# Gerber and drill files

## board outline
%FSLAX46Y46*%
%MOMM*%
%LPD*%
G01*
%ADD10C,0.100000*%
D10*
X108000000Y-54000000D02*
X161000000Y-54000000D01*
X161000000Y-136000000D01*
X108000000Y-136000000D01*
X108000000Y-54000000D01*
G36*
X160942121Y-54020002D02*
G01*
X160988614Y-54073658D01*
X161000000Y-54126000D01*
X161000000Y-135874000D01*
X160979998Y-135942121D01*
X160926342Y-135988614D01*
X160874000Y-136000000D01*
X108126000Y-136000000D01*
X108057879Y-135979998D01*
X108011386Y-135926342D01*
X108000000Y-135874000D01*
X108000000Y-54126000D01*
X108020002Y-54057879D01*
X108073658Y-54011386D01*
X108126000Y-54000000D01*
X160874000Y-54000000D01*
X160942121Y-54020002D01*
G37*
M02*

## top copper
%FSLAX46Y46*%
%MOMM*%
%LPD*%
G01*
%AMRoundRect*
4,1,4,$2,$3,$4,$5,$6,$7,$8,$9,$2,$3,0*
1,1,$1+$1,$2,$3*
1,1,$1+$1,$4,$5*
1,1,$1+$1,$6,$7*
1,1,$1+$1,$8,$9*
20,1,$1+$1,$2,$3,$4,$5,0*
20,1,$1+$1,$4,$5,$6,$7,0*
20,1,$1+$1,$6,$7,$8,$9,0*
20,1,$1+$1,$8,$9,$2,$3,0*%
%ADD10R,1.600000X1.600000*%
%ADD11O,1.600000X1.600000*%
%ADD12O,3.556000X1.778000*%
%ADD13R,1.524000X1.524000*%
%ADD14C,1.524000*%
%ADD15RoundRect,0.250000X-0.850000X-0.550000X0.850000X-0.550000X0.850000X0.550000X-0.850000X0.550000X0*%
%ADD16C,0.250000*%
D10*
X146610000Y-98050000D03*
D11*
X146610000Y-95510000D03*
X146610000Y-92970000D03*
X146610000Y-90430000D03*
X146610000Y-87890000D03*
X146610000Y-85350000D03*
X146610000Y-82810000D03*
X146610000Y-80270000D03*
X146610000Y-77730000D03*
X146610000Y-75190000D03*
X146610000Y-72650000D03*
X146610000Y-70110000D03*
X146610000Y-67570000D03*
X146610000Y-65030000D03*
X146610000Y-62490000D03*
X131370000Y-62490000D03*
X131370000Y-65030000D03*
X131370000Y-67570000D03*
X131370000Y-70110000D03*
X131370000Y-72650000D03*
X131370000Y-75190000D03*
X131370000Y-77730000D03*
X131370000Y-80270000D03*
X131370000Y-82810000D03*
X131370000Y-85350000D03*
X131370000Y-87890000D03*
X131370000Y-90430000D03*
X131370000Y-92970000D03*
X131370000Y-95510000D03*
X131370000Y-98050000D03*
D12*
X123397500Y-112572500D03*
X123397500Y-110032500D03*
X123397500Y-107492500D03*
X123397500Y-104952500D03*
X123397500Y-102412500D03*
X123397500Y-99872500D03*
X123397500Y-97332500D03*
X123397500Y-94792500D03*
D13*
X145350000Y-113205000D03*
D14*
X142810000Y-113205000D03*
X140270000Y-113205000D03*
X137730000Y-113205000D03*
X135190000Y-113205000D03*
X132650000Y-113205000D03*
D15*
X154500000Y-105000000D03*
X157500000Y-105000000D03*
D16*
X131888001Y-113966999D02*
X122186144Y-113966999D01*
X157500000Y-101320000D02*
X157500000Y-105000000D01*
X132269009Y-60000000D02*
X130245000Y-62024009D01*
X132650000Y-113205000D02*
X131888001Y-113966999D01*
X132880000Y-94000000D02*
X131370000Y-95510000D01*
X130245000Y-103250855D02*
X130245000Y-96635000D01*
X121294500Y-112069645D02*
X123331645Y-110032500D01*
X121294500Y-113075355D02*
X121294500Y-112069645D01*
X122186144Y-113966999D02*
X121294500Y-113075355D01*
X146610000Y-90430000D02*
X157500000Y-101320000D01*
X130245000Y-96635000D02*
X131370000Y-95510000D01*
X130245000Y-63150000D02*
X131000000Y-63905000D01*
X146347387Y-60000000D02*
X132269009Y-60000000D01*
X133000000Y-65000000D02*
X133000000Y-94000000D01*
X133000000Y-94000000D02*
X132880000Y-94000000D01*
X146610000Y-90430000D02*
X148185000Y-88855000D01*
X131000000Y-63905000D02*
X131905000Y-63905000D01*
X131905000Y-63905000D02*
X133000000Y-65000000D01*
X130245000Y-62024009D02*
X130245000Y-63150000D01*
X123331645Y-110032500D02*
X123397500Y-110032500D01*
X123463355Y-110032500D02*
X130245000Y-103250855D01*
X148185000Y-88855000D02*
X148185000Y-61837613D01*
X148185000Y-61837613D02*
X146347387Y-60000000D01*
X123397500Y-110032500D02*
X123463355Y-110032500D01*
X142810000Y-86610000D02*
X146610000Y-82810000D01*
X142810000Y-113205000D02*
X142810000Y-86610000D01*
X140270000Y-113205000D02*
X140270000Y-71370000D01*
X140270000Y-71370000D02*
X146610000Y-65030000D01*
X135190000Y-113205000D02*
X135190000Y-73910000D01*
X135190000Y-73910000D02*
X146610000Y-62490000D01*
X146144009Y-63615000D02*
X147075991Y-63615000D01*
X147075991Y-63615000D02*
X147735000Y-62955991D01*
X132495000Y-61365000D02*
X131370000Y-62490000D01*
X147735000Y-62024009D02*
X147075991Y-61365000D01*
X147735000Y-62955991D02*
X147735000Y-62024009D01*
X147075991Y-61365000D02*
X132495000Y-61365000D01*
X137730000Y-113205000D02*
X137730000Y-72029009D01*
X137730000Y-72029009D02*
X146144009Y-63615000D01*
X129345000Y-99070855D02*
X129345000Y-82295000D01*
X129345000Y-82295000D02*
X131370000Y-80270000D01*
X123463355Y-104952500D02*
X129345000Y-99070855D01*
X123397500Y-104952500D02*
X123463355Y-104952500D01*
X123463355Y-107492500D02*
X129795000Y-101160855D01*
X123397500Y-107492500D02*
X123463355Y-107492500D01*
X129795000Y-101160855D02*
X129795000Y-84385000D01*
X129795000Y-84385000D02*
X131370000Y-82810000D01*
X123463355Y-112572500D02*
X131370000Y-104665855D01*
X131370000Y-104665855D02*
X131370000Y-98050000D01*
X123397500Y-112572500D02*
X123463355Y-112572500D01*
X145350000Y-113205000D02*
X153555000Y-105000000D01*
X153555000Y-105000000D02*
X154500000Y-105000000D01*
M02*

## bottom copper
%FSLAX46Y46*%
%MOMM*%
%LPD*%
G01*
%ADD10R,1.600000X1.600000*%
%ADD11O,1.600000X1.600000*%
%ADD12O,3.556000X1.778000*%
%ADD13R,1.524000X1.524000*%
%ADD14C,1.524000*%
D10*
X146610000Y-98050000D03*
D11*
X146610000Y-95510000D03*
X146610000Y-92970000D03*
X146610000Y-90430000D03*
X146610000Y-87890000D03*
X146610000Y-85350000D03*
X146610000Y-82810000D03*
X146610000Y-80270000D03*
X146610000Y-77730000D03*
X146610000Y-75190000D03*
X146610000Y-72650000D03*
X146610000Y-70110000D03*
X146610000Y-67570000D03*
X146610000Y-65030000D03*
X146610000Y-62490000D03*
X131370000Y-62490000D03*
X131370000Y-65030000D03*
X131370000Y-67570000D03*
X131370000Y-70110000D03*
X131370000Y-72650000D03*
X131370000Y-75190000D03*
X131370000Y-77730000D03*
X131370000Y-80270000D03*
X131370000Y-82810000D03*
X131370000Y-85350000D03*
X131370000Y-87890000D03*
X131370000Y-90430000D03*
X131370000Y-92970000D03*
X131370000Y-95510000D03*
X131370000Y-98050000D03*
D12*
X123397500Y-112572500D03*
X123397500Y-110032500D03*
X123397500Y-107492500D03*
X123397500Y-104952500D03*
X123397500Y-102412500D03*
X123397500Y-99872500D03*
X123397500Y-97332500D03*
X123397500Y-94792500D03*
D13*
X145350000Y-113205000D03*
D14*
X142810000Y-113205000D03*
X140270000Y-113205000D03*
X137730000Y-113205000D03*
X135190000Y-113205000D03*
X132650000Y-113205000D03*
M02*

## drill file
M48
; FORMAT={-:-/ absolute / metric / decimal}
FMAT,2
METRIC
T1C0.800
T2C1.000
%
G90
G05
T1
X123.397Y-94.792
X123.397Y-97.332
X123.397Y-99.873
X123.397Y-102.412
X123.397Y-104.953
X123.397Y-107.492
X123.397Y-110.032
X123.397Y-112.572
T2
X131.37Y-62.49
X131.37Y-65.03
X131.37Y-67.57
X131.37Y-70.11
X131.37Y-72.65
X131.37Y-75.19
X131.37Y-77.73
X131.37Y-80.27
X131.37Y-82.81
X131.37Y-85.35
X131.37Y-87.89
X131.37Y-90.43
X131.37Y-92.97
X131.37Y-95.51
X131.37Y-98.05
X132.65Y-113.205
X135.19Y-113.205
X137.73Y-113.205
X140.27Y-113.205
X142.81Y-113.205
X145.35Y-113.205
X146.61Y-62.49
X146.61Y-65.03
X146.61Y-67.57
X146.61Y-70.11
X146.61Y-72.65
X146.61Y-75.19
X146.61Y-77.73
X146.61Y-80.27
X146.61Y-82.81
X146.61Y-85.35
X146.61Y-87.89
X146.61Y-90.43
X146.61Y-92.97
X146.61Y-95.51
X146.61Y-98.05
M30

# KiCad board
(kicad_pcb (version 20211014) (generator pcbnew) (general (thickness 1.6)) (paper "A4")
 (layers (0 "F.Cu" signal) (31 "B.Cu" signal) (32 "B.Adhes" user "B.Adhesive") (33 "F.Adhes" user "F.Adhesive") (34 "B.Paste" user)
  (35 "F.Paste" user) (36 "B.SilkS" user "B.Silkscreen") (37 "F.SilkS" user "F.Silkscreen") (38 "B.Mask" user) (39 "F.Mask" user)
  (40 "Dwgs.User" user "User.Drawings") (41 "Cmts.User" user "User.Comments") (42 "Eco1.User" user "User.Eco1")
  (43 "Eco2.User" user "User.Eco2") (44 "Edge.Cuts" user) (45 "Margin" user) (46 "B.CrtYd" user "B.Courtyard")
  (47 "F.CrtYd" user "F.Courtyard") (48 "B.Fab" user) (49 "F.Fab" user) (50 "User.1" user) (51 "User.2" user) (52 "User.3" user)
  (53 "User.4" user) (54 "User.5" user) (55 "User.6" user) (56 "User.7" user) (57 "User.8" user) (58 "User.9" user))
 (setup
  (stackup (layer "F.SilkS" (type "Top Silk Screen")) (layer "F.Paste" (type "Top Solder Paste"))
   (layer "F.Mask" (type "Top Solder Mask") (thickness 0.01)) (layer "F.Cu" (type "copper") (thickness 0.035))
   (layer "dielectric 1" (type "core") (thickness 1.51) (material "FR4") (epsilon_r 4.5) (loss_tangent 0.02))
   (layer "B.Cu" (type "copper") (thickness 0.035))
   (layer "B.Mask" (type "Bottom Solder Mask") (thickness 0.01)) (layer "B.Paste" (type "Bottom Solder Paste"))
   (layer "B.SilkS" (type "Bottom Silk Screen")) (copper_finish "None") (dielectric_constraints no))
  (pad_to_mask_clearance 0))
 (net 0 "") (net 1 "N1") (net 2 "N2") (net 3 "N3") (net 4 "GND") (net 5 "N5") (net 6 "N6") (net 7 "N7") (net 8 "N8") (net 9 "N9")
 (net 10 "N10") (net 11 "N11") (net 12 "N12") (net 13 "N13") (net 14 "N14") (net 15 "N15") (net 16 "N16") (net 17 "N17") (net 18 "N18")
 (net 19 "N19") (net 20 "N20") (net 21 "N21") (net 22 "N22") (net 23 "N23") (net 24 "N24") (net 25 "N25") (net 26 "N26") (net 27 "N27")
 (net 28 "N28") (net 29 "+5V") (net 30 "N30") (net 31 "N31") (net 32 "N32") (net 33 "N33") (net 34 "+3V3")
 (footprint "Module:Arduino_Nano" (layer "F.Cu") (at 146.61 98.05 180)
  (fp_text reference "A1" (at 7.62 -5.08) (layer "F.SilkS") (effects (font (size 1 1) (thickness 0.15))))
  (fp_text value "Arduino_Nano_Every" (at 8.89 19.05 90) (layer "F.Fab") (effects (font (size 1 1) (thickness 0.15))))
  (pad "1" thru_hole rect (at 0 0 180) (size 1.6 1.6) (drill 1) (layers *.Cu *.Mask) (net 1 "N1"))
  (pad "2" thru_hole oval (at 0 2.54 180) (size 1.6 1.6) (drill 1) (layers *.Cu *.Mask) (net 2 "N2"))
  (pad "3" thru_hole oval (at 0 5.08 180) (size 1.6 1.6) (drill 1) (layers *.Cu *.Mask) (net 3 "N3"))
  (pad "4" thru_hole oval (at 0 7.62 180) (size 1.6 1.6) (drill 1) (layers *.Cu *.Mask) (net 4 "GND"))
  (pad "5" thru_hole oval (at 0 10.16 180) (size 1.6 1.6) (drill 1) (layers *.Cu *.Mask) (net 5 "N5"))
  (pad "6" thru_hole oval (at 0 12.7 180) (size 1.6 1.6) (drill 1) (layers *.Cu *.Mask) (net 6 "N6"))
  (pad "7" thru_hole oval (at 0 15.24 180) (size 1.6 1.6) (drill 1) (layers *.Cu *.Mask) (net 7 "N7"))
  (pad "8" thru_hole oval (at 0 17.78 180) (size 1.6 1.6) (drill 1) (layers *.Cu *.Mask) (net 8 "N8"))
  (pad "9" thru_hole oval (at 0 20.32 180) (size 1.6 1.6) (drill 1) (layers *.Cu *.Mask) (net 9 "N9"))
  (pad "10" thru_hole oval (at 0 22.86 180) (size 1.6 1.6) (drill 1) (layers *.Cu *.Mask) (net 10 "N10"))
  (pad "11" thru_hole oval (at 0 25.4 180) (size 1.6 1.6) (drill 1) (layers *.Cu *.Mask) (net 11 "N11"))
  (pad "12" thru_hole oval (at 0 27.94 180) (size 1.6 1.6) (drill 1) (layers *.Cu *.Mask) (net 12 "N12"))
  (pad "13" thru_hole oval (at 0 30.48 180) (size 1.6 1.6) (drill 1) (layers *.Cu *.Mask) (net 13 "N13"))
  (pad "14" thru_hole oval (at 0 33.02 180) (size 1.6 1.6) (drill 1) (layers *.Cu *.Mask) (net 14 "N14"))
  (pad "15" thru_hole oval (at 0 35.56 180) (size 1.6 1.6) (drill 1) (layers *.Cu *.Mask) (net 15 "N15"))
  (pad "16" thru_hole oval (at 15.24 35.56 180) (size 1.6 1.6) (drill 1) (layers *.Cu *.Mask) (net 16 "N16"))
  (pad "17" thru_hole oval (at 15.24 33.02 180) (size 1.6 1.6) (drill 1) (layers *.Cu *.Mask) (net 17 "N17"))
  (pad "18" thru_hole oval (at 15.24 30.48 180) (size 1.6 1.6) (drill 1) (layers *.Cu *.Mask) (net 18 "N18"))
  (pad "19" thru_hole oval (at 15.24 27.94 180) (size 1.6 1.6) (drill 1) (layers *.Cu *.Mask) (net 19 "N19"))
  (pad "20" thru_hole oval (at 15.24 25.4 180) (size 1.6 1.6) (drill 1) (layers *.Cu *.Mask) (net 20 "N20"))
  (pad "21" thru_hole oval (at 15.24 22.86 180) (size 1.6 1.6) (drill 1) (layers *.Cu *.Mask) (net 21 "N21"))
  (pad "22" thru_hole oval (at 15.24 20.32 180) (size 1.6 1.6) (drill 1) (layers *.Cu *.Mask) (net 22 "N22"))
  (pad "23" thru_hole oval (at 15.24 17.78 180) (size 1.6 1.6) (drill 1) (layers *.Cu *.Mask) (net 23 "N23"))
  (pad "24" thru_hole oval (at 15.24 15.24 180) (size 1.6 1.6) (drill 1) (layers *.Cu *.Mask) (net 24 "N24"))
  (pad "25" thru_hole oval (at 15.24 12.7 180) (size 1.6 1.6) (drill 1) (layers *.Cu *.Mask) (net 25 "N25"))
  (pad "26" thru_hole oval (at 15.24 10.16 180) (size 1.6 1.6) (drill 1) (layers *.Cu *.Mask) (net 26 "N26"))
  (pad "27" thru_hole oval (at 15.24 7.62 180) (size 1.6 1.6) (drill 1) (layers *.Cu *.Mask) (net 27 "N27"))
  (pad "28" thru_hole oval (at 15.24 5.08 180) (size 1.6 1.6) (drill 1) (layers *.Cu *.Mask) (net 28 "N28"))
  (pad "29" thru_hole oval (at 15.24 2.54 180) (size 1.6 1.6) (drill 1) (layers *.Cu *.Mask) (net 4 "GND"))
  (pad "30" thru_hole oval (at 15.24 0 180) (size 1.6 1.6) (drill 1) (layers *.Cu *.Mask) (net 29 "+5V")))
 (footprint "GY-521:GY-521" (layer "F.Cu") (at 114.5075 103.6825 180)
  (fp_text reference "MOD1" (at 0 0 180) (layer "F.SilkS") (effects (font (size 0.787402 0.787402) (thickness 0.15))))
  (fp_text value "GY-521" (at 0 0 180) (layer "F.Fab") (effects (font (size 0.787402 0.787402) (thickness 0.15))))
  (pad "1" thru_hole oval locked (at -8.89 -8.89 180) (size 3.556 1.778) (drill 0.8) (layers *.Cu *.Mask) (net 29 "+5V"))
  (pad "2" thru_hole oval locked (at -8.89 -6.35 180) (size 3.556 1.778) (drill 0.8) (layers *.Cu *.Mask) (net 4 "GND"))
  (pad "3" thru_hole oval locked (at -8.89 -3.81 180) (size 3.556 1.778) (drill 0.8) (layers *.Cu *.Mask) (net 24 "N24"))
  (pad "4" thru_hole oval locked (at -8.89 -1.27 180) (size 3.556 1.778) (drill 0.8) (layers *.Cu *.Mask) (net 23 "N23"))
  (pad "5" thru_hole oval locked (at -8.89 1.27 180) (size 3.556 1.778) (drill 0.8) (layers *.Cu *.Mask) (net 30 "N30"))
  (pad "6" thru_hole oval locked (at -8.89 3.81 180) (size 3.556 1.778) (drill 0.8) (layers *.Cu *.Mask) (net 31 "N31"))
  (pad "7" thru_hole oval locked (at -8.89 6.35 180) (size 3.556 1.778) (drill 0.8) (layers *.Cu *.Mask) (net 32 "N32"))
  (pad "8" thru_hole oval locked (at -8.89 8.89 180) (size 3.556 1.778) (drill 0.8) (layers *.Cu *.Mask) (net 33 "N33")))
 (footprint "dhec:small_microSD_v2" (layer "F.Cu") (at 138.365 110.03)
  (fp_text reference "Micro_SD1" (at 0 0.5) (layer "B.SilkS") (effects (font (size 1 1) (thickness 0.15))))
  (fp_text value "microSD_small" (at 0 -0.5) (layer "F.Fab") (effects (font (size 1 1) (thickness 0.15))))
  (pad "1" thru_hole rect locked (at 6.985 3.175) (size 1.524 1.524) (drill 1) (layers *.Cu *.Mask) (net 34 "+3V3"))
  (pad "2" thru_hole circle locked (at 4.445 3.175) (size 1.524 1.524) (drill 1) (layers *.Cu *.Mask) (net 7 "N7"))
  (pad "3" thru_hole circle locked (at 1.905 3.175) (size 1.524 1.524) (drill 1) (layers *.Cu *.Mask) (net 14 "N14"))
  (pad "4" thru_hole circle locked (at -0.635 3.175) (size 1.524 1.524) (drill 1) (layers *.Cu *.Mask) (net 16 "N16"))
  (pad "5" thru_hole circle locked (at -3.175 3.175) (size 1.524 1.524) (drill 1) (layers *.Cu *.Mask) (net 15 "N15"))
  (pad "6" thru_hole circle locked (at -5.715 3.175) (size 1.524 1.524) (drill 1) (layers *.Cu *.Mask) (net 4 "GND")))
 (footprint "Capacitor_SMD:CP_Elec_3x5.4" (layer "F.Cu") (at 156 105)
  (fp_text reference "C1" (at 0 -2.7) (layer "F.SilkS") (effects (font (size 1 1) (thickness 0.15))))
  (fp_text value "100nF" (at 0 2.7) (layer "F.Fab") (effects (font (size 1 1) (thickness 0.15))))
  (pad "1" smd roundrect (at -1.5 0) (size 2.2 1.6) (layers "F.Cu" "F.Paste" "F.Mask") (roundrect_rratio 0.15625) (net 34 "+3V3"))
  (pad "2" smd roundrect (at 1.5 0) (size 2.2 1.6) (layers "F.Cu" "F.Paste" "F.Mask") (roundrect_rratio 0.15625) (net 4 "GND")))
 (gr_rect (start 108 54) (end 161 136) (layer "Edge.Cuts") (width 0.1) (fill none))
 (segment (start 131.888001 113.966999) (end 122.186144 113.966999) (width 0.25) (layer "F.Cu") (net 4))
 (segment (start 157.5 101.32) (end 157.5 105) (width 0.25) (layer "F.Cu") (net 4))
 (segment (start 132.269009 60) (end 130.245 62.024009) (width 0.25) (layer "F.Cu") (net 4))
 (segment (start 132.65 113.205) (end 131.888001 113.966999) (width 0.25) (layer "F.Cu") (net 4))
 (segment (start 132.88 94) (end 131.37 95.51) (width 0.25) (layer "F.Cu") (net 4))
 (segment (start 130.245 103.250855) (end 130.245 96.635) (width 0.25) (layer "F.Cu") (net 4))
 (segment (start 121.2945 112.069645) (end 123.331645 110.0325) (width 0.25) (layer "F.Cu") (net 4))
 (segment (start 121.2945 113.075355) (end 121.2945 112.069645) (width 0.25) (layer "F.Cu") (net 4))
 (segment (start 122.186144 113.966999) (end 121.2945 113.075355) (width 0.25) (layer "F.Cu") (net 4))
 (segment (start 146.61 90.43) (end 157.5 101.32) (width 0.25) (layer "F.Cu") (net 4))
 (segment (start 130.245 96.635) (end 131.37 95.51) (width 0.25) (layer "F.Cu") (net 4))
 (segment (start 130.245 63.15) (end 131 63.905) (width 0.25) (layer "F.Cu") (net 4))
 (segment (start 146.347387 60) (end 132.269009 60) (width 0.25) (layer "F.Cu") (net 4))
 (segment (start 133 65) (end 133 94) (width 0.25) (layer "F.Cu") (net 4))
 (segment (start 133 94) (end 132.88 94) (width 0.25) (layer "F.Cu") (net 4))
 (segment (start 146.61 90.43) (end 148.185 88.855) (width 0.25) (layer "F.Cu") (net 4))
 (segment (start 131 63.905) (end 131.905 63.905) (width 0.25) (layer "F.Cu") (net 4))
 (segment (start 131.905 63.905) (end 133 65) (width 0.25) (layer "F.Cu") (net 4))
 (segment (start 130.245 62.024009) (end 130.245 63.15) (width 0.25) (layer "F.Cu") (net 4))
 (segment (start 123.331645 110.0325) (end 123.3975 110.0325) (width 0.25) (layer "F.Cu") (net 4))
 (segment (start 123.463355 110.0325) (end 130.245 103.250855) (width 0.25) (layer "F.Cu") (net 4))
 (segment (start 148.185 88.855) (end 148.185 61.837613) (width 0.25) (layer "F.Cu") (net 4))
 (segment (start 148.185 61.837613) (end 146.347387 60) (width 0.25) (layer "F.Cu") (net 4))
 (segment (start 123.3975 110.0325) (end 123.463355 110.0325) (width 0.25) (layer "F.Cu") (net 4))
 (segment (start 142.81 86.61) (end 146.61 82.81) (width 0.25) (layer "F.Cu") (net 7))
 (segment (start 142.81 113.205) (end 142.81 86.61) (width 0.25) (layer "F.Cu") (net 7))
 (segment (start 140.27 113.205) (end 140.27 71.37) (width 0.25) (layer "F.Cu") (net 14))
 (segment (start 140.27 71.37) (end 146.61 65.03) (width 0.25) (layer "F.Cu") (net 14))
 (segment (start 135.19 113.205) (end 135.19 73.91) (width 0.25) (layer "F.Cu") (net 15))
 (segment (start 135.19 73.91) (end 146.61 62.49) (width 0.25) (layer "F.Cu") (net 15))
 (segment (start 146.144009 63.615) (end 147.075991 63.615) (width 0.25) (layer "F.Cu") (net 16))
 (segment (start 147.075991 63.615) (end 147.735 62.955991) (width 0.25) (layer "F.Cu") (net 16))
 (segment (start 132.495 61.365) (end 131.37 62.49) (width 0.25) (layer "F.Cu") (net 16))
 (segment (start 147.735 62.024009) (end 147.075991 61.365) (width 0.25) (layer "F.Cu") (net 16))
 (segment (start 147.735 62.955991) (end 147.735 62.024009) (width 0.25) (layer "F.Cu") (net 16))
 (segment (start 147.075991 61.365) (end 132.495 61.365) (width 0.25) (layer "F.Cu") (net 16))
 (segment (start 137.73 113.205) (end 137.73 72.029009) (width 0.25) (layer "F.Cu") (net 16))
 (segment (start 137.73 72.029009) (end 146.144009 63.615) (width 0.25) (layer "F.Cu") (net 16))
 (segment (start 129.345 99.070855) (end 129.345 82.295) (width 0.25) (layer "F.Cu") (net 23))
 (segment (start 129.345 82.295) (end 131.37 80.27) (width 0.25) (layer "F.Cu") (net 23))
 (segment (start 123.463355 104.9525) (end 129.345 99.070855) (width 0.25) (layer "F.Cu") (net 23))
 (segment (start 123.3975 104.9525) (end 123.463355 104.9525) (width 0.25) (layer "F.Cu") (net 23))
 (segment (start 123.463355 107.4925) (end 129.795 101.160855) (width 0.25) (layer "F.Cu") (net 24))
 (segment (start 123.3975 107.4925) (end 123.463355 107.4925) (width 0.25) (layer "F.Cu") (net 24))
 (segment (start 129.795 101.160855) (end 129.795 84.385) (width 0.25) (layer "F.Cu") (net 24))
 (segment (start 129.795 84.385) (end 131.37 82.81) (width 0.25) (layer "F.Cu") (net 24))
 (segment (start 123.463355 112.5725) (end 131.37 104.665855) (width 0.25) (layer "F.Cu") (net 29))
 (segment (start 131.37 104.665855) (end 131.37 98.05) (width 0.25) (layer "F.Cu") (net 29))
 (segment (start 123.3975 112.5725) (end 123.463355 112.5725) (width 0.25) (layer "F.Cu") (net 29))
 (segment (start 145.35 113.205) (end 153.555 105) (width 0.25) (layer "F.Cu") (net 34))
 (segment (start 153.555 105) (end 154.5 105) (width 0.25) (layer "F.Cu") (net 34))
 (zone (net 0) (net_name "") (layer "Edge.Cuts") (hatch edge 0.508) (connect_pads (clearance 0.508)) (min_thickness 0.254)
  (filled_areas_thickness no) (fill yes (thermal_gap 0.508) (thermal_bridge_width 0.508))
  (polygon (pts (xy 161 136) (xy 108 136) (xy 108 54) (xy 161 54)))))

